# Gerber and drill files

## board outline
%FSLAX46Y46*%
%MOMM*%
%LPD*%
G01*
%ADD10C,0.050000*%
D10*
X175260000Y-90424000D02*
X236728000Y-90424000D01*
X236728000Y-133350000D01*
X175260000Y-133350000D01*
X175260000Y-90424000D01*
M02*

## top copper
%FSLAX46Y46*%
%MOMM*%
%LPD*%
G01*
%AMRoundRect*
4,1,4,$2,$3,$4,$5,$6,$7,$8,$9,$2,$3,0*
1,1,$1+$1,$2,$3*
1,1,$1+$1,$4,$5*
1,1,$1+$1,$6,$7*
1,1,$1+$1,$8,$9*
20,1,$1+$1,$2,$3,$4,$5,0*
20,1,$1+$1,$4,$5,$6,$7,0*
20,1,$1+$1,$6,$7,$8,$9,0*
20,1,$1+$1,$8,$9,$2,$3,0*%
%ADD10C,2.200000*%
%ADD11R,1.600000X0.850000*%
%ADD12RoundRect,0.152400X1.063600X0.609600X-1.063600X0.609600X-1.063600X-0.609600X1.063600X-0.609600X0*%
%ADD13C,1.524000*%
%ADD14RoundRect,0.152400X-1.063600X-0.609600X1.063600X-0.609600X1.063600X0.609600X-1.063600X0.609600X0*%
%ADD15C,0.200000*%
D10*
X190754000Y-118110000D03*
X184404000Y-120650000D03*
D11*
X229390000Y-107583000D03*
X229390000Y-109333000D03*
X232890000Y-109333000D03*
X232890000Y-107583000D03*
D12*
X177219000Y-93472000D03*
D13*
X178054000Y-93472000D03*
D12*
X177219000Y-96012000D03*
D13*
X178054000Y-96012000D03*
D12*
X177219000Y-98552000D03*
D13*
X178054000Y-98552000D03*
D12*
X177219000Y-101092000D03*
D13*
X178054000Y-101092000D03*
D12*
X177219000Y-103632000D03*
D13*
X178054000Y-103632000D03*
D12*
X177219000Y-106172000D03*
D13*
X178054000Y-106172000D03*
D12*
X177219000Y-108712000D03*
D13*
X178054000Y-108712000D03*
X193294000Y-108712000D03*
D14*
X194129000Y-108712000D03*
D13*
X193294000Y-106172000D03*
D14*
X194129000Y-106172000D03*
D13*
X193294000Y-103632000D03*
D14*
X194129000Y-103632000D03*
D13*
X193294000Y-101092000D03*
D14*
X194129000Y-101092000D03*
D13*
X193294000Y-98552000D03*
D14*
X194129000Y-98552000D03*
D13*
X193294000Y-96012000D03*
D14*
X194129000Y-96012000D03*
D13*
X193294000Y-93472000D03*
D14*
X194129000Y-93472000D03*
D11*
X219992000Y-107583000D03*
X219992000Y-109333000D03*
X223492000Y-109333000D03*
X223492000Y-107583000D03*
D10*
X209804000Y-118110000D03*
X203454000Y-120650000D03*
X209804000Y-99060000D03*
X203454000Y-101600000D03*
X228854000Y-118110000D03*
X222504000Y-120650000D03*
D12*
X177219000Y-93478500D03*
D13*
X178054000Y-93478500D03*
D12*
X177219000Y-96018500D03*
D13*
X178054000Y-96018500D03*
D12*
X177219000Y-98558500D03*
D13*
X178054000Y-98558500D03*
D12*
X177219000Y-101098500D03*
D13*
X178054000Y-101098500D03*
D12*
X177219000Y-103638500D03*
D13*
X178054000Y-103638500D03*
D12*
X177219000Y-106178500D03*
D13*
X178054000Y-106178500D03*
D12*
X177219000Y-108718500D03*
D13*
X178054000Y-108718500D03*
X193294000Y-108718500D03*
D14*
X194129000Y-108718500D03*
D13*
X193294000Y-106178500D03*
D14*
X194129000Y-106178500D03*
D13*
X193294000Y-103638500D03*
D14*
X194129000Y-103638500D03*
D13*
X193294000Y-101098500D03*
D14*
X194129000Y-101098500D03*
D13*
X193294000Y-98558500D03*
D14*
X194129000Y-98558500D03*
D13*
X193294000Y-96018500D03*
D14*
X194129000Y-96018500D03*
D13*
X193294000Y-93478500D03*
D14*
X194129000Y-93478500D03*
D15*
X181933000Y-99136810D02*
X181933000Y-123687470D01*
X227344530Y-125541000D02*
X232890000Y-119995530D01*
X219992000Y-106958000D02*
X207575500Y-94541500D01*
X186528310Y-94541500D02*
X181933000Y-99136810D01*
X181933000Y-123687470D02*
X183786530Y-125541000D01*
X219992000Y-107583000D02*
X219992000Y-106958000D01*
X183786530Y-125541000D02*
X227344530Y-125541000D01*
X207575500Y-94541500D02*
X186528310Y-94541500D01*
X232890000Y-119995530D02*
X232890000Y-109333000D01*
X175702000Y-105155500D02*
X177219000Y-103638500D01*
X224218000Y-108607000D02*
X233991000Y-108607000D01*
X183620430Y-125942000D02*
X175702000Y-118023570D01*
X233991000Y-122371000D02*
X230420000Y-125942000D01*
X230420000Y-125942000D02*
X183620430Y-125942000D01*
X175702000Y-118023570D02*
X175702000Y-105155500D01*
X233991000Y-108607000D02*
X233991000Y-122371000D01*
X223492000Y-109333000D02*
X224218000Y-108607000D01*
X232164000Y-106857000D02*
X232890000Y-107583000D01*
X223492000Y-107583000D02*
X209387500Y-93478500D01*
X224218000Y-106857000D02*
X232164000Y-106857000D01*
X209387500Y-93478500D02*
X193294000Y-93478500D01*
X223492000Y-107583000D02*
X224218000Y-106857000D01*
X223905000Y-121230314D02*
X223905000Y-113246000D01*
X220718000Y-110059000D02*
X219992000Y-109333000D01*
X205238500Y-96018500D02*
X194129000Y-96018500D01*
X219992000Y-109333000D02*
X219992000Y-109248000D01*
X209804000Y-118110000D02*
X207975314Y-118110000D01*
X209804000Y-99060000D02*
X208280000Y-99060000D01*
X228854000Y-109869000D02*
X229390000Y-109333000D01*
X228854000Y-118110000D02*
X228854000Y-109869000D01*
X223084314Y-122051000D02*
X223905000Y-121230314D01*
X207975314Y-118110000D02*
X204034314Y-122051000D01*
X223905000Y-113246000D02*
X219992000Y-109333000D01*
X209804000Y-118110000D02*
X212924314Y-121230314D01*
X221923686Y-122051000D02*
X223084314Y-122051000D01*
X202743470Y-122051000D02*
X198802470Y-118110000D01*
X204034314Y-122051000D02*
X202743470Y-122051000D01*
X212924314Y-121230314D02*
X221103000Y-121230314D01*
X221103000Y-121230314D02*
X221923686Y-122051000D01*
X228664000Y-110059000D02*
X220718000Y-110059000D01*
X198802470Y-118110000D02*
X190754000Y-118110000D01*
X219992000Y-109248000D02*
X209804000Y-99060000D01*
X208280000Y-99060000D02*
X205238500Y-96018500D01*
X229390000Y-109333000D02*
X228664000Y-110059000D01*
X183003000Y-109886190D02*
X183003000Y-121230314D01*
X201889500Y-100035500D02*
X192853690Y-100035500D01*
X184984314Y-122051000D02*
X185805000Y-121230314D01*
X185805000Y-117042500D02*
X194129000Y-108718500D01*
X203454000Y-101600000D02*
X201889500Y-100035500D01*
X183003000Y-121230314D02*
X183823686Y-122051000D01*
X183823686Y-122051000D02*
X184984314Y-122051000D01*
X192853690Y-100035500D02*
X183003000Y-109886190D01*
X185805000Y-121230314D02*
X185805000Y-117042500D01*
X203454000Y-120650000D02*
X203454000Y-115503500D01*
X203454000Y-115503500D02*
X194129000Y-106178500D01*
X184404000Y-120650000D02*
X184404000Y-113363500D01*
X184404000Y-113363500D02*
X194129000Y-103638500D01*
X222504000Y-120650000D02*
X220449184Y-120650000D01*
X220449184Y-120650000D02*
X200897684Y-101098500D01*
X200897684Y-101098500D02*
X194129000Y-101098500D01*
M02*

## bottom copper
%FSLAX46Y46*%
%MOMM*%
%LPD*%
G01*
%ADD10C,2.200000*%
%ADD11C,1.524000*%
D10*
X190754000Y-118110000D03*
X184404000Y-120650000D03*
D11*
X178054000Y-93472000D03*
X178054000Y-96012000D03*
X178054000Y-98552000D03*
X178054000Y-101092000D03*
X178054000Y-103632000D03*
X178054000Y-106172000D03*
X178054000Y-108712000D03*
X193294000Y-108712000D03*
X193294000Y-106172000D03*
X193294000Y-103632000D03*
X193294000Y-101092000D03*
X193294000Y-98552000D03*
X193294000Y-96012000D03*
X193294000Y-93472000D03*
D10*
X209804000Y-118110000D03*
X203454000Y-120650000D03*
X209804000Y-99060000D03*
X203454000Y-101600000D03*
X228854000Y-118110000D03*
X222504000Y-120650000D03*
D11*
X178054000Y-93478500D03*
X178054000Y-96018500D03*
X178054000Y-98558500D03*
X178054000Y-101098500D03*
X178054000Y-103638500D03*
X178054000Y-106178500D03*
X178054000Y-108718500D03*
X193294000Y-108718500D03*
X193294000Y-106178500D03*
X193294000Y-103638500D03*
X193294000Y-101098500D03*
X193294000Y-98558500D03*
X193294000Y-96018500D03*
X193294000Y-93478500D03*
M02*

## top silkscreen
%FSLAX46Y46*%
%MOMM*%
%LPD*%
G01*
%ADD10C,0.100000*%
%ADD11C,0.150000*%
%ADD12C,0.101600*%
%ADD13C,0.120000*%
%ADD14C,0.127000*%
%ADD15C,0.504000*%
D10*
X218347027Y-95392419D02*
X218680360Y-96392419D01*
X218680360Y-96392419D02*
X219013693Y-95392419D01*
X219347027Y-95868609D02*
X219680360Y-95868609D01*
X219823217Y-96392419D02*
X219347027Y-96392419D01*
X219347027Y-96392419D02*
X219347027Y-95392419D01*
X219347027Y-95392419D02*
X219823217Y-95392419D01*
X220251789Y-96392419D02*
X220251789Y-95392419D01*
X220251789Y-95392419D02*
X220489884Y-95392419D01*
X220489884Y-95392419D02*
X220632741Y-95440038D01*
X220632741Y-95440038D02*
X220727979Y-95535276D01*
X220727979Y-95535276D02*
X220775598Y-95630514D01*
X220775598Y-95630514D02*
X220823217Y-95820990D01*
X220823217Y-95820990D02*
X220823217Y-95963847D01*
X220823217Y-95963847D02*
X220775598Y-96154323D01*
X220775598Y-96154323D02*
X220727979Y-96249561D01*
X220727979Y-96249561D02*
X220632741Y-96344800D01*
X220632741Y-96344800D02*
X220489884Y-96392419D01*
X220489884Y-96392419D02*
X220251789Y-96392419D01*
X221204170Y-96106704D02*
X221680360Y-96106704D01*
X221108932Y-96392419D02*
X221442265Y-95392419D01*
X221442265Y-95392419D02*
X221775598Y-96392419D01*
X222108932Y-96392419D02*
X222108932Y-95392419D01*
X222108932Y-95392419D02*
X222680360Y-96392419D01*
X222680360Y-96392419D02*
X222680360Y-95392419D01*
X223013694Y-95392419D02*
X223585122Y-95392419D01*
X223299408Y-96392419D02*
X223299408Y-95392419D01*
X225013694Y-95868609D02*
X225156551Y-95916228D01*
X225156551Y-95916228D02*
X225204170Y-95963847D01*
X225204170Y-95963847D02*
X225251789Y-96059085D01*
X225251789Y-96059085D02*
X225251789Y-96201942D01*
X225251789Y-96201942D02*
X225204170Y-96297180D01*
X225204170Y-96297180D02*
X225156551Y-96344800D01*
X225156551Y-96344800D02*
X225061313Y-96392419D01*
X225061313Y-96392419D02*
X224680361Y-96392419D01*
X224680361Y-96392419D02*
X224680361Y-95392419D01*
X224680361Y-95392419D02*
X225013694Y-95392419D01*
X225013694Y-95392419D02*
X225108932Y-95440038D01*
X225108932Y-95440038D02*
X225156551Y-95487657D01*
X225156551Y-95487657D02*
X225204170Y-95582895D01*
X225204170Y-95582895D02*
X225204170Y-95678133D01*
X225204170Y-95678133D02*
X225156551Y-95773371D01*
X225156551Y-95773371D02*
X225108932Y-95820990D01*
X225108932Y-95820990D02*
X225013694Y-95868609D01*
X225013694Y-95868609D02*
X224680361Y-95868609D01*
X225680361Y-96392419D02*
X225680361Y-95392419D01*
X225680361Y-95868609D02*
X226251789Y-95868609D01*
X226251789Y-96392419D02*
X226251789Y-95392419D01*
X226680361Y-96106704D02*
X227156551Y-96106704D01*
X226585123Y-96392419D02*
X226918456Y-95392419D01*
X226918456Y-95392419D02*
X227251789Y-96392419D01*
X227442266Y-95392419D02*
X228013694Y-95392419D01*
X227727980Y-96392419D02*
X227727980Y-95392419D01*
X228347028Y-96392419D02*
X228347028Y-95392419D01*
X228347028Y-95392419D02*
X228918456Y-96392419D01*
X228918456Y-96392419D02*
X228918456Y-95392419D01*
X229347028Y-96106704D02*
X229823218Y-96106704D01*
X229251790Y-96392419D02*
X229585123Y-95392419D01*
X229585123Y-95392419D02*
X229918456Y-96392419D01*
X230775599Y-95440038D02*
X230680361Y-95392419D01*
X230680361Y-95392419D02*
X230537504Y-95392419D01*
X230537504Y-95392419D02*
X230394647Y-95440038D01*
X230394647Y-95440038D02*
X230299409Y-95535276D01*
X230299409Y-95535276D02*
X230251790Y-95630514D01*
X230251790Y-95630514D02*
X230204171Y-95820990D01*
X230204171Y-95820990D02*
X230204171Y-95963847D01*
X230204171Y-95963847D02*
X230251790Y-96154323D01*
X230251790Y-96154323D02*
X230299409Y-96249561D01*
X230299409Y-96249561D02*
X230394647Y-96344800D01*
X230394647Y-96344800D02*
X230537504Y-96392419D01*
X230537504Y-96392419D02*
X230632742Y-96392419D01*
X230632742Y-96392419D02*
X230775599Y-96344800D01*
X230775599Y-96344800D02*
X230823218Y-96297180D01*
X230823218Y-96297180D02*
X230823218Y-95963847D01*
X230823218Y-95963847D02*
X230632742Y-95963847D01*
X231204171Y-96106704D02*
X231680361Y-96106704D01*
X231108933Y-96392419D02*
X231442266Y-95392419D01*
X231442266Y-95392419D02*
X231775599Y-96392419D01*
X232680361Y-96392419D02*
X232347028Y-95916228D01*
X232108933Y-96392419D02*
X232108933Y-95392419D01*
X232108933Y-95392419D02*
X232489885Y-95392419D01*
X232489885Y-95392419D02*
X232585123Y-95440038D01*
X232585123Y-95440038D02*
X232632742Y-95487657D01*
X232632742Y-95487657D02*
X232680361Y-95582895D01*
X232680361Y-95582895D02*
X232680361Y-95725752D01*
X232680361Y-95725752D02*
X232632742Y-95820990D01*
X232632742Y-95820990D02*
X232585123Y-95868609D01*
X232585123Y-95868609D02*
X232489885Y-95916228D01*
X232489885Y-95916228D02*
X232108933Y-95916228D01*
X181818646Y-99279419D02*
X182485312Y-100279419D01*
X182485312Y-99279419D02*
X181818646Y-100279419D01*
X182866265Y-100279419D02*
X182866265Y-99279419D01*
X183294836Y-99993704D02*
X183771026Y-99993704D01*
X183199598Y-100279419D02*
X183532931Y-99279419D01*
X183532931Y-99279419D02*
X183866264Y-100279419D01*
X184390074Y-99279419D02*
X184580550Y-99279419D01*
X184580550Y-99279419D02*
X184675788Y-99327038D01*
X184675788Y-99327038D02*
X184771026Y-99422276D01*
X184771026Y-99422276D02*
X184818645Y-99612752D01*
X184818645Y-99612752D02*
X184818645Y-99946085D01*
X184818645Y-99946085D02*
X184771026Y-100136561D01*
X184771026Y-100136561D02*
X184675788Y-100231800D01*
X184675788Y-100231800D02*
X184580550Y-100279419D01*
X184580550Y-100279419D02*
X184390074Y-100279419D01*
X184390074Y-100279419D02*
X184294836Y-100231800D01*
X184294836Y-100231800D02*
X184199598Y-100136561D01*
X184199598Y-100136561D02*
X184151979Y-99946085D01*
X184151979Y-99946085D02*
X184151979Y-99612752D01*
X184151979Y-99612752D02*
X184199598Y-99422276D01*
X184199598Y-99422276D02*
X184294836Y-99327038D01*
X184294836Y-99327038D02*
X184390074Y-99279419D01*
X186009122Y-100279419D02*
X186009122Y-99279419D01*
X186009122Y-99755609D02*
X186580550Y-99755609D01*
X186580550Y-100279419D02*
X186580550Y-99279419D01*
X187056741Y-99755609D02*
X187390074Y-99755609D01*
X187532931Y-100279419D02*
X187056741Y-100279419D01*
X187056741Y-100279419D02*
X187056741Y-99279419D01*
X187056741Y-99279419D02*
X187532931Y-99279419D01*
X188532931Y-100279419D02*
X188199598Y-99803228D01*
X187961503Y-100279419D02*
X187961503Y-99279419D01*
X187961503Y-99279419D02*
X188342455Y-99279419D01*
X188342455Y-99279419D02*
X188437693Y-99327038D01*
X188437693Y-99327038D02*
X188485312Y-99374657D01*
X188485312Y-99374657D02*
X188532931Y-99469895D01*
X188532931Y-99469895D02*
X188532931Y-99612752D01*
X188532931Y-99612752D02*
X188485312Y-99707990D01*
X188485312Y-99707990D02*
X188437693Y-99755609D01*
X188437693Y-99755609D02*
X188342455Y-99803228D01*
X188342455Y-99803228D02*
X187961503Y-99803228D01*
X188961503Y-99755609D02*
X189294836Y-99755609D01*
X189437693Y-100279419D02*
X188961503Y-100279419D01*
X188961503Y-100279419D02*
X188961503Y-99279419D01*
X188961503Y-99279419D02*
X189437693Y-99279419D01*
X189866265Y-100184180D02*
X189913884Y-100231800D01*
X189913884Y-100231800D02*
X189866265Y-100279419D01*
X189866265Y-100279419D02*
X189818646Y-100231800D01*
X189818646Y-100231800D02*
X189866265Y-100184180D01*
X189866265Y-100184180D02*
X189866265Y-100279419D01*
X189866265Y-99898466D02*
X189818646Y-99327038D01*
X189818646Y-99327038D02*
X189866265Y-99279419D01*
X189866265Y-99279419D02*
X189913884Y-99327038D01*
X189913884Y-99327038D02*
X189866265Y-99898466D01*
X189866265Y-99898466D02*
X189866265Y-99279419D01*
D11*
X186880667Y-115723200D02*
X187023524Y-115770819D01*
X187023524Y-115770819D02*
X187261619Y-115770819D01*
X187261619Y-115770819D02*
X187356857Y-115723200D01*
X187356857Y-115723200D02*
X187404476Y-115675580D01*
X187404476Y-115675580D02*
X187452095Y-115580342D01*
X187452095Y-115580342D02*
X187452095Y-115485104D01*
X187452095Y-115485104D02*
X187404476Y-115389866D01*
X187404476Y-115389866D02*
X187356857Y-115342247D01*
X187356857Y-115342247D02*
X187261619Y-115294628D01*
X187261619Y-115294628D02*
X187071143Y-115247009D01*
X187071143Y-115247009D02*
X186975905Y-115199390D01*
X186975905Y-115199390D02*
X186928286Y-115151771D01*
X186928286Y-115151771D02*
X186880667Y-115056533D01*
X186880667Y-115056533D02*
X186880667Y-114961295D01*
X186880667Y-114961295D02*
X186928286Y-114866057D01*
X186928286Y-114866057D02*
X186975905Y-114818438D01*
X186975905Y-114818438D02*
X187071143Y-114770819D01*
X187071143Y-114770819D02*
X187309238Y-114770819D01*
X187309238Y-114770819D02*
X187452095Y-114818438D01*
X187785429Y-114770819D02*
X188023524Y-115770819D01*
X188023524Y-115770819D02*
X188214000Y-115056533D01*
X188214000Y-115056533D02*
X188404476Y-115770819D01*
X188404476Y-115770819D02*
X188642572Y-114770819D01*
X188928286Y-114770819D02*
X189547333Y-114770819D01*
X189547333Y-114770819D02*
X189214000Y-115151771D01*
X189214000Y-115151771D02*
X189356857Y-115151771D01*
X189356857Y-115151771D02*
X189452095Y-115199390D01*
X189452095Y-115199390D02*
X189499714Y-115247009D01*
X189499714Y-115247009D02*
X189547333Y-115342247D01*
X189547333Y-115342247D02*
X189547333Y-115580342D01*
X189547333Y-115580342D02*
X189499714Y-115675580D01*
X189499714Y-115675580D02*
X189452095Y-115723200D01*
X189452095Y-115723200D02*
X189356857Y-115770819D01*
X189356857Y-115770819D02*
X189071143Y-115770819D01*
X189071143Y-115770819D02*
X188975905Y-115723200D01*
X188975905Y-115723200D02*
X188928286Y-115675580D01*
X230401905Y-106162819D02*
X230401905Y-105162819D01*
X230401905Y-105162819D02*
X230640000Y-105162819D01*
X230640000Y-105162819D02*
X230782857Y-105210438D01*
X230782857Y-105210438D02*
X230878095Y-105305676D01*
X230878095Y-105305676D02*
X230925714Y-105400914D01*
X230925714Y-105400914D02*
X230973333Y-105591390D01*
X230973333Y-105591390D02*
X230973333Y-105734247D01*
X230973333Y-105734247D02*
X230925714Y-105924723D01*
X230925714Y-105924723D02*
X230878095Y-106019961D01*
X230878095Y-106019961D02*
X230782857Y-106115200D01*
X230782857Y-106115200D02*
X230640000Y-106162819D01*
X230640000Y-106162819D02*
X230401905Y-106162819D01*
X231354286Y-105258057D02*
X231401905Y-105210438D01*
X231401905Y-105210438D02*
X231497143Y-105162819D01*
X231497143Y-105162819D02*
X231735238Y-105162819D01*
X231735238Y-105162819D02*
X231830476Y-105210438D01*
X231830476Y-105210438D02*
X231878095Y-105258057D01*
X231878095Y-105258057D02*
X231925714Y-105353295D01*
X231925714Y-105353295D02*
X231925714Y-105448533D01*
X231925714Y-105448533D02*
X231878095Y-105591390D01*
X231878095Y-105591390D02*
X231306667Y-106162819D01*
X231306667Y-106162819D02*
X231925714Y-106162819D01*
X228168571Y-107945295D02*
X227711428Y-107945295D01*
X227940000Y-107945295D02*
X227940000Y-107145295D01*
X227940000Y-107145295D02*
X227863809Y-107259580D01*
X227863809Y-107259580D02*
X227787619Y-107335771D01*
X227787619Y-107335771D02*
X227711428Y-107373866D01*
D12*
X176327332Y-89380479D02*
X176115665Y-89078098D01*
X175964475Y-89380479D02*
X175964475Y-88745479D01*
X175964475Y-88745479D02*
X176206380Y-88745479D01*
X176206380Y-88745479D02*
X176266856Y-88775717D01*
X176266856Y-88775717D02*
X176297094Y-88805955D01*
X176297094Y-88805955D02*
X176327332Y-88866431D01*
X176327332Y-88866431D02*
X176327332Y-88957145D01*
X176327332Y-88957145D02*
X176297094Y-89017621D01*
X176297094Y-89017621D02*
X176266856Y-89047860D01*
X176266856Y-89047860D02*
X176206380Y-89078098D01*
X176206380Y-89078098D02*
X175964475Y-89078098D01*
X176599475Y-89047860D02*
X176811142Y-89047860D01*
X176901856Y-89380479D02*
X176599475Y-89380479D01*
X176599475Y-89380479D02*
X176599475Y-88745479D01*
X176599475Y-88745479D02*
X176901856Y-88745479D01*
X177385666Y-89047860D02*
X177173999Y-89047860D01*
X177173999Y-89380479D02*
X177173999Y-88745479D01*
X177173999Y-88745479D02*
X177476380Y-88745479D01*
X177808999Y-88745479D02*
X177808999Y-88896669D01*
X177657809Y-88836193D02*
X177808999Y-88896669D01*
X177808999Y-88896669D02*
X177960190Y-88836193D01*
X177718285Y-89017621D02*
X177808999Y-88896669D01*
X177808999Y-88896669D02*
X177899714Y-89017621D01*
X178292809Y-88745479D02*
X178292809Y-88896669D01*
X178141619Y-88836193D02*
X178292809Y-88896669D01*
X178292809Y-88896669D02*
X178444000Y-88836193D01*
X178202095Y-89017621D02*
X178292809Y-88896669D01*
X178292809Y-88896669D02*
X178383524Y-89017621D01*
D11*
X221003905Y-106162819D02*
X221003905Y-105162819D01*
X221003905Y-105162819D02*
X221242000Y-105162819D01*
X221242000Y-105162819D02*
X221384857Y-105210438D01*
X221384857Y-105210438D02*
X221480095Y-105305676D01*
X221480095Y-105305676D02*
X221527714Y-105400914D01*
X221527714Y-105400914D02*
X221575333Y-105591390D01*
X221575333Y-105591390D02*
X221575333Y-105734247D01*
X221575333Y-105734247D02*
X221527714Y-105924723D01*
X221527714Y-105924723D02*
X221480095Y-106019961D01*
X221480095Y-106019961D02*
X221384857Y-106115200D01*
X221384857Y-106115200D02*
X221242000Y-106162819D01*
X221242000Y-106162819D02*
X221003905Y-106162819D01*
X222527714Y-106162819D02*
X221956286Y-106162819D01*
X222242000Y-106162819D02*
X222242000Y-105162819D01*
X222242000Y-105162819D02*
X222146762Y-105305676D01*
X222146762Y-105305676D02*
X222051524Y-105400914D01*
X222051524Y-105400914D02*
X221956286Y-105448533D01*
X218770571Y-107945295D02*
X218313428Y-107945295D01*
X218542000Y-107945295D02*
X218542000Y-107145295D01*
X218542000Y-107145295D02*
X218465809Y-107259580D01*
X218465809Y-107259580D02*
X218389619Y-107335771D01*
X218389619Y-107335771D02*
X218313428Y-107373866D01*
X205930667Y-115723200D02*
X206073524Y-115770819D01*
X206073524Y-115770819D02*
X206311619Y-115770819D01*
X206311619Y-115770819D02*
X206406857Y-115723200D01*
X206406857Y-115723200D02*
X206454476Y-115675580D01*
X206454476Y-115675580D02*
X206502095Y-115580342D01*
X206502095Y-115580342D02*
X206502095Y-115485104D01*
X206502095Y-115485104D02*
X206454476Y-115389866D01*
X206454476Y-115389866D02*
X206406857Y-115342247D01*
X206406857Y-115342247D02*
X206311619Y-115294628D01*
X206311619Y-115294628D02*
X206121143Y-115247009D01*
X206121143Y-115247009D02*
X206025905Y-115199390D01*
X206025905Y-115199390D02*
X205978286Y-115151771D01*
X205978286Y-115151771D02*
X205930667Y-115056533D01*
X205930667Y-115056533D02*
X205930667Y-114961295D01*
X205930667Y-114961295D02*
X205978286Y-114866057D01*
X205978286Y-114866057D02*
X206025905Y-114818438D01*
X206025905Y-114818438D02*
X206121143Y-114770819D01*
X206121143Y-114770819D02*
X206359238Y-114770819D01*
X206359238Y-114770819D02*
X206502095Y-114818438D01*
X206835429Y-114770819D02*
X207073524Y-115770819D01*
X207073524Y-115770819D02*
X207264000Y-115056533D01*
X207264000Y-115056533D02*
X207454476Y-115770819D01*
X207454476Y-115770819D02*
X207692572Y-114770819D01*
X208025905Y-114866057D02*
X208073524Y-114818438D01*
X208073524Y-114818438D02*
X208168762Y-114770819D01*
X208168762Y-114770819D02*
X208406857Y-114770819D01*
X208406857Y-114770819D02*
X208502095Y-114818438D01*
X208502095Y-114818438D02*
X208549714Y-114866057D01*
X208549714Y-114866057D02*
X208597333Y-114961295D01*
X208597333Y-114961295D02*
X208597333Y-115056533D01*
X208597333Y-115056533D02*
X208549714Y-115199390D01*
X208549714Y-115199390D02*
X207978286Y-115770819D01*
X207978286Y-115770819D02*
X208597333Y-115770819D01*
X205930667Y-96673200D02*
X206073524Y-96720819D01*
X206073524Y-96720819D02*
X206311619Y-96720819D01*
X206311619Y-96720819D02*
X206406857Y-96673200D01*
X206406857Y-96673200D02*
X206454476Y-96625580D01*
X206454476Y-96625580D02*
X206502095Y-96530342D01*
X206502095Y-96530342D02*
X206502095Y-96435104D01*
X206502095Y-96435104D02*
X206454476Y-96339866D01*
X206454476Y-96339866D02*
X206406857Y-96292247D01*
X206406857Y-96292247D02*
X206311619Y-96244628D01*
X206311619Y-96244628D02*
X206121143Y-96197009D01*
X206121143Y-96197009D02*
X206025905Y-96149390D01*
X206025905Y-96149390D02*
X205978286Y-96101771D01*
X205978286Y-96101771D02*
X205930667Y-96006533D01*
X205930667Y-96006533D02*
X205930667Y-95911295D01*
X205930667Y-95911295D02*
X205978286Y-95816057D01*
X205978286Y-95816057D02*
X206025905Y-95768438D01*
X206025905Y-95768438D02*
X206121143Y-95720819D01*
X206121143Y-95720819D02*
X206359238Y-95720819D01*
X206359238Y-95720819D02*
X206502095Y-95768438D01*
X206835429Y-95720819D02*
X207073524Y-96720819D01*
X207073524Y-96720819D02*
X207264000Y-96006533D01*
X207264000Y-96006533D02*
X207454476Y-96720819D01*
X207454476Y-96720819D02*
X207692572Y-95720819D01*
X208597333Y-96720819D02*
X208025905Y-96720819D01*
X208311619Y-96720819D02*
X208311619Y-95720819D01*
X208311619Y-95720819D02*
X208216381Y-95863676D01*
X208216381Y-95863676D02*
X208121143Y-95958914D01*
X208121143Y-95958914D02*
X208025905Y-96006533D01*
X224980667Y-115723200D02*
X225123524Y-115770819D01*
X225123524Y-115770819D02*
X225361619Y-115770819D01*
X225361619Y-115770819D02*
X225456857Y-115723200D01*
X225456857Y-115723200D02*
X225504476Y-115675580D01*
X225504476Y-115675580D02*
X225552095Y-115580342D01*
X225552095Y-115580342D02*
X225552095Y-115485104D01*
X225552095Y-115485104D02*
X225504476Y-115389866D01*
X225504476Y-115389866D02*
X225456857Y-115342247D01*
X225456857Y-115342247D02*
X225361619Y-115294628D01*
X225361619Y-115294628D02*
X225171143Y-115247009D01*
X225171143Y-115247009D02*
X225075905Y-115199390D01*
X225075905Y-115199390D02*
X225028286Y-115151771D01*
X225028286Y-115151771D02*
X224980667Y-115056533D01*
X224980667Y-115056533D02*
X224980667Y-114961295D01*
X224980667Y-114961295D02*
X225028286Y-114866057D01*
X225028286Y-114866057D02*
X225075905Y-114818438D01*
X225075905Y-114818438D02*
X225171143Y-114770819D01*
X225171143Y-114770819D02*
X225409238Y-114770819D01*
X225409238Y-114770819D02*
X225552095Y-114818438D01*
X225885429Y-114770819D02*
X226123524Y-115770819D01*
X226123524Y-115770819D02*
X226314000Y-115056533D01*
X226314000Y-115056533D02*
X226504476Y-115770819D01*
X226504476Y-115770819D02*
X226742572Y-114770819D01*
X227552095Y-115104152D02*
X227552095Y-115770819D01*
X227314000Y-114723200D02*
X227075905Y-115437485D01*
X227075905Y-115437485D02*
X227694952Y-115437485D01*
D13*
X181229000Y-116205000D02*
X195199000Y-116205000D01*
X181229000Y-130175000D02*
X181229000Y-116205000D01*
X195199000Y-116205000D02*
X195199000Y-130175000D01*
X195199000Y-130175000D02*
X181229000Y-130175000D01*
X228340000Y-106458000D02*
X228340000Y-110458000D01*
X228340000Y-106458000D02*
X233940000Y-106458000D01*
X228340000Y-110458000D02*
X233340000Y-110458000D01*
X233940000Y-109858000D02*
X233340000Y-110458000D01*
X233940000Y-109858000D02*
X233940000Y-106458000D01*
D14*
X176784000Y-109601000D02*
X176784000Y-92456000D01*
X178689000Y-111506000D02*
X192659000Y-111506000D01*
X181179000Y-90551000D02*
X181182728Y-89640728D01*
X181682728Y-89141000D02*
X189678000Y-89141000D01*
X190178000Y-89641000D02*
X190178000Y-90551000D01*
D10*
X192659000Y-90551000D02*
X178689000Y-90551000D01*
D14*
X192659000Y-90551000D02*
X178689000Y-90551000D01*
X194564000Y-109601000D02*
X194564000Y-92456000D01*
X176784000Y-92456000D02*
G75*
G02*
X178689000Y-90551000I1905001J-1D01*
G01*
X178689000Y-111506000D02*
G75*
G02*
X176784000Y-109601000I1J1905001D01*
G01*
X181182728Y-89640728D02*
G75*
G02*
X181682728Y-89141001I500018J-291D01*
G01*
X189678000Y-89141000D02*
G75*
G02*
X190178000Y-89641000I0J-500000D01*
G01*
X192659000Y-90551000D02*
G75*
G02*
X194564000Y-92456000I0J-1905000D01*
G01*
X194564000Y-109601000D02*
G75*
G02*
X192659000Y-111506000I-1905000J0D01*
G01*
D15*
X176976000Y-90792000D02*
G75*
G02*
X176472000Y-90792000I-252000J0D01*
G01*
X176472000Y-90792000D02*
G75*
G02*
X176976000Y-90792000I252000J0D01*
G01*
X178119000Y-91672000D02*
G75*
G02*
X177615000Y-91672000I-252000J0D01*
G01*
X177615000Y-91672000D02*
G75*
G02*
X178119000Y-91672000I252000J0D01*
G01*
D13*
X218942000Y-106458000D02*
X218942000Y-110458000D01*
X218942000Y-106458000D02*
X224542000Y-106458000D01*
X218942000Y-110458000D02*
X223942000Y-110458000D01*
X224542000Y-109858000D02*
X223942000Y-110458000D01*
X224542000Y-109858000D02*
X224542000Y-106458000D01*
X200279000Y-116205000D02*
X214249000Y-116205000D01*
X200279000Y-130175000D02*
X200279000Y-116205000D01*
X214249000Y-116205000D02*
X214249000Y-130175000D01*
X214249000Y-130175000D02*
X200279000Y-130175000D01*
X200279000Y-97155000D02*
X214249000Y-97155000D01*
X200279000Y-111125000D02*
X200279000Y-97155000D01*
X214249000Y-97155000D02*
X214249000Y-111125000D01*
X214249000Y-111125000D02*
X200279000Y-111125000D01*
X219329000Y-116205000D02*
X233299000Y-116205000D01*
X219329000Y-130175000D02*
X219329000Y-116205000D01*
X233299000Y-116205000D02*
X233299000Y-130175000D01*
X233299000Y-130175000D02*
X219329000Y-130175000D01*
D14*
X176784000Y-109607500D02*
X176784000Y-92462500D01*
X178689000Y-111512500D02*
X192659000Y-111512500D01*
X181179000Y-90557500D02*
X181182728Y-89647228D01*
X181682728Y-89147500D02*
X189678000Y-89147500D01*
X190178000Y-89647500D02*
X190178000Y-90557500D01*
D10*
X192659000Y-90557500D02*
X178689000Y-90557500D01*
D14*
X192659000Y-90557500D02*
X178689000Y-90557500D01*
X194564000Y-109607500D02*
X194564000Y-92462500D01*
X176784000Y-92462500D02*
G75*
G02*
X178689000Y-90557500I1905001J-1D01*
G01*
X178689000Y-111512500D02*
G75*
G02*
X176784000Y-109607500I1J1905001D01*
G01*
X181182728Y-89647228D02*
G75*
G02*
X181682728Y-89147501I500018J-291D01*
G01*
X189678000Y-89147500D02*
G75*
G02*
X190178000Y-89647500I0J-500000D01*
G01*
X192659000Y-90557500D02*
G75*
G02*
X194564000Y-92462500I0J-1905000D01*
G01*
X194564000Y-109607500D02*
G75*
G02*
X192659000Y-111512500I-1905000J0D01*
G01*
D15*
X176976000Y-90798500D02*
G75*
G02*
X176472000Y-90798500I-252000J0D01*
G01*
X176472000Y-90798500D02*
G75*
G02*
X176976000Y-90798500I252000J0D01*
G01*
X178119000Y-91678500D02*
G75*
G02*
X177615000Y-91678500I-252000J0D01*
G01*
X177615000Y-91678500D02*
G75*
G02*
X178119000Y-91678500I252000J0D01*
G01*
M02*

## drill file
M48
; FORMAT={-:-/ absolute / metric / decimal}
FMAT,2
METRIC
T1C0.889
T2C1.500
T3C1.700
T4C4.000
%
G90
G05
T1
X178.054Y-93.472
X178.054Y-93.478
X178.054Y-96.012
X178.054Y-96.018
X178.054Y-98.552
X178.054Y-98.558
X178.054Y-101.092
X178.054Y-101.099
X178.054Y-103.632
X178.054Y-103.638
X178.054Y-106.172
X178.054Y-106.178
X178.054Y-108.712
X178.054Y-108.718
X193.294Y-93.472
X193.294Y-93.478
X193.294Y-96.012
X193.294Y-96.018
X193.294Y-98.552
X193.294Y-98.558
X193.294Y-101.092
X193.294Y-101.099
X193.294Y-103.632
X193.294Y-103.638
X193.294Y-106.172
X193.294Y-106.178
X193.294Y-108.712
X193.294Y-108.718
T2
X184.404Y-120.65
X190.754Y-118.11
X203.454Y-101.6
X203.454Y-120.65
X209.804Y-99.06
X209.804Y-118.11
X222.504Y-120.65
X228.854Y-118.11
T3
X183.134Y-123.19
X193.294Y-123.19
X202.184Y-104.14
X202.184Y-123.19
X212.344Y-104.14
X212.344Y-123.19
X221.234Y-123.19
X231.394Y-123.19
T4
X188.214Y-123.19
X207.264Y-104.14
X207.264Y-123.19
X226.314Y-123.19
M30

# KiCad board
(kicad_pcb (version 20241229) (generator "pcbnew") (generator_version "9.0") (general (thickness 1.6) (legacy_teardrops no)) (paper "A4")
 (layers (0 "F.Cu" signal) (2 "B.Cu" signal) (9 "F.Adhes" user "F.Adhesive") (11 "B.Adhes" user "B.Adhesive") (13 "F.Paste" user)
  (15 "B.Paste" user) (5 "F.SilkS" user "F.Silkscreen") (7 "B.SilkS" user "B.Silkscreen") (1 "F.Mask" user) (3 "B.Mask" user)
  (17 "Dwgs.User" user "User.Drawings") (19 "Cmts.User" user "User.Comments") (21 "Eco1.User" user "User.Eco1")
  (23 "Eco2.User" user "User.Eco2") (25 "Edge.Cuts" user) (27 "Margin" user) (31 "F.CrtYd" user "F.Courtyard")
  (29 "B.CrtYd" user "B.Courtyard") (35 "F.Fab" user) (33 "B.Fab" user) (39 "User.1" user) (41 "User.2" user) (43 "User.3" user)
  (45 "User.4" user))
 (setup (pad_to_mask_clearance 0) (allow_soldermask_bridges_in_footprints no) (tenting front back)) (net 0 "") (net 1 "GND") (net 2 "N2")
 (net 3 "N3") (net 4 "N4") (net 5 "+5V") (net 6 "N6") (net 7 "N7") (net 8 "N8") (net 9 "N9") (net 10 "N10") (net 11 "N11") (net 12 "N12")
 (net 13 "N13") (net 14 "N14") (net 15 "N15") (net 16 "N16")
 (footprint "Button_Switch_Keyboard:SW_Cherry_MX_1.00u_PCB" (layer "F.Cu") (at 190.754 118.11)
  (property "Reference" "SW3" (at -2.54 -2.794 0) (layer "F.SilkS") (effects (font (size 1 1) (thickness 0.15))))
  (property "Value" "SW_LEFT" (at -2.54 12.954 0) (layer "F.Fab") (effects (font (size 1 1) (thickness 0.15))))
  (fp_line (start -9.525 -1.905) (end 4.445 -1.905) (stroke (width 0.12) (type solid)) (layer "F.SilkS"))
  (fp_line (start -9.525 12.065) (end -9.525 -1.905) (stroke (width 0.12) (type solid)) (layer "F.SilkS"))
  (fp_line (start 4.445 -1.905) (end 4.445 12.065) (stroke (width 0.12) (type solid)) (layer "F.SilkS"))
  (fp_line (start 4.445 12.065) (end -9.525 12.065) (stroke (width 0.12) (type solid)) (layer "F.SilkS"))
  (pad "" np_thru_hole circle (at -7.62 5.08) (size 1.7 1.7) (drill 1.7) (layers "*.Cu" "*.Mask"))
  (pad "" np_thru_hole circle (at -2.54 5.08) (size 4 4) (drill 4) (layers "*.Cu" "*.Mask"))
  (pad "" np_thru_hole circle (at 2.54 5.08) (size 1.7 1.7) (drill 1.7) (layers "*.Cu" "*.Mask"))
  (pad "1" thru_hole circle (at 0 0) (size 2.2 2.2) (drill 1.5) (layers "*.Cu" "*.Mask") (remove_unused_layers no) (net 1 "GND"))
  (pad "2" thru_hole circle (at -6.35 2.54) (size 2.2 2.2) (drill 1.5) (layers "*.Cu" "*.Mask") (remove_unused_layers no) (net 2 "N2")))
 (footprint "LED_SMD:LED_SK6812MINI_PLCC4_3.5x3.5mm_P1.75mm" (layer "F.Cu") (at 231.14 108.458)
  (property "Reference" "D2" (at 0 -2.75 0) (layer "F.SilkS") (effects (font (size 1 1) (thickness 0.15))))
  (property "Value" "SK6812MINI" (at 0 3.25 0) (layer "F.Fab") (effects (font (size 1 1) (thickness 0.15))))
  (fp_line (start -2.8 -2) (end -2.8 2) (stroke (width 0.12) (type default)) (layer "F.SilkS"))
  (fp_line (start -2.8 -2) (end 2.8 -2) (stroke (width 0.12) (type solid)) (layer "F.SilkS"))
  (fp_line (start -2.8 2) (end 2.2 2) (stroke (width 0.12) (type solid)) (layer "F.SilkS"))
  (fp_line (start 2.8 1.4) (end 2.2 2) (stroke (width 0.12) (type default)) (layer "F.SilkS"))
  (fp_line (start 2.8 1.4) (end 2.8 -2) (stroke (width 0.12) (type solid)) (layer "F.SilkS"))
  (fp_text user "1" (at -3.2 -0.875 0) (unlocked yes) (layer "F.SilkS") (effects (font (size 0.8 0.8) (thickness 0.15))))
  (pad "1" smd rect (at -1.75 -0.875) (size 1.6 0.85) (layers "F.Cu" "F.Mask" "F.Paste") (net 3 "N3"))
  (pad "2" smd rect (at -1.75 0.875) (size 1.6 0.85) (layers "F.Cu" "F.Mask" "F.Paste") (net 1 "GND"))
  (pad "3" smd rect (at 1.75 0.875) (size 1.6 0.85) (layers "F.Cu" "F.Mask" "F.Paste") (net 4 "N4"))
  (pad "4" smd rect (at 1.75 -0.875) (size 1.6 0.85) (layers "F.Cu" "F.Mask" "F.Paste") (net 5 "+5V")))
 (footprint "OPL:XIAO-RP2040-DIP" (layer "F.Cu") (at 185.674 101.092)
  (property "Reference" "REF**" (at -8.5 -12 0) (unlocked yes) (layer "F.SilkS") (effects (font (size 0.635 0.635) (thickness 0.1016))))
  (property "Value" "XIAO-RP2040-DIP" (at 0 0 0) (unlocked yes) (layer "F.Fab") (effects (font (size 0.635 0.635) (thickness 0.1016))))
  (fp_line (start -8.89 8.509) (end -8.89 -8.636) (stroke (width 0.127) (type solid)) (layer "F.SilkS"))
  (fp_line (start -6.985 10.414) (end 6.985 10.414) (stroke (width 0.127) (type solid)) (layer "F.SilkS"))
  (fp_line (start -4.495 -10.541) (end -4.491272 -11.451272) (stroke (width 0.127) (type solid)) (layer "F.SilkS"))
  (fp_line (start -3.991272 -11.951) (end 4.004 -11.951) (stroke (width 0.127) (type solid)) (layer "F.SilkS"))
  (fp_line (start 4.504 -11.451) (end 4.504 -10.541) (stroke (width 0.127) (type solid)) (layer "F.SilkS"))
  (fp_line (start 6.985 -10.541) (end -6.985 -10.541) (stroke (width 0.1) (type solid)) (layer "F.SilkS"))
  (fp_line (start 6.985 -10.541) (end -6.985 -10.541) (stroke (width 0.127) (type solid)) (layer "F.SilkS"))
  (fp_line (start 8.89 8.509) (end 8.89 -8.636) (stroke (width 0.127) (type solid)) (layer "F.SilkS"))
  (fp_arc (start -8.89 -8.636) (mid -8.332038 -9.983038) (end -6.985 -10.541) (stroke (width 0.127) (type solid)) (layer "F.SilkS"))
  (fp_arc (start -6.985 10.414) (mid -8.332038 9.856038) (end -8.89 8.509) (stroke (width 0.127) (type solid)) (layer "F.SilkS"))
  (fp_arc (start -4.491272 -11.451272) (mid -4.344728 -11.80464) (end -3.991272 -11.951) (stroke (width 0.127) (type default))
   (layer "F.SilkS"))
  (fp_arc (start 4.004 -11.951) (mid 4.357553 -11.804553) (end 4.504 -11.451) (stroke (width 0.127) (type default)) (layer "F.SilkS"))
  (fp_arc (start 6.985 -10.541) (mid 8.332038 -9.983038) (end 8.89 -8.636) (stroke (width 0.127) (type solid)) (layer "F.SilkS"))
  (fp_arc (start 8.89 8.509) (mid 8.332038 9.856038) (end 6.985 10.414) (stroke (width 0.127) (type solid)) (layer "F.SilkS"))
  (fp_circle (center -8.95 -10.3) (end -8.95 -10.554) (stroke (width 0.5) (type solid)) (fill yes) (layer "F.SilkS"))
  (fp_circle (center -7.807 -9.42) (end -7.807 -9.674) (stroke (width 0.5) (type solid)) (fill yes) (layer "F.SilkS"))
  (pad "1" smd roundrect (at -8.455 -7.62 180) (size 2.432 1.524) (layers "F.Cu" "F.Mask") (roundrect_rratio 0.1) (thermal_bridge_angle 45))
  (pad "1" thru_hole circle (at -7.62 -7.62 180) (size 1.524 1.524) (drill 0.889) (layers "*.Cu" "*.Mask") (remove_unused_layers no))
  (pad "2" smd roundrect (at -8.455 -5.08 180) (size 2.432 1.524) (layers "F.Cu" "F.Mask") (roundrect_rratio 0.1) (thermal_bridge_angle 45))
  (pad "2" thru_hole circle (at -7.62 -5.08 180) (size 1.524 1.524) (drill 0.889) (layers "*.Cu" "*.Mask") (remove_unused_layers no))
  (pad "3" smd roundrect (at -8.455 -2.54 180) (size 2.432 1.524) (layers "F.Cu" "F.Mask") (roundrect_rratio 0.1) (thermal_bridge_angle 45))
  (pad "3" thru_hole circle (at -7.62 -2.54 180) (size 1.524 1.524) (drill 0.889) (layers "*.Cu" "*.Mask") (remove_unused_layers no))
  (pad "4" smd roundrect (at -8.455 0 180) (size 2.432 1.524) (layers "F.Cu" "F.Mask") (roundrect_rratio 0.1) (thermal_bridge_angle 45))
  (pad "4" thru_hole circle (at -7.62 0 180) (size 1.524 1.524) (drill 0.889) (layers "*.Cu" "*.Mask") (remove_unused_layers no))
  (pad "5" smd roundrect (at -8.455 2.54 180) (size 2.432 1.524) (layers "F.Cu" "F.Mask") (roundrect_rratio 0.1) (thermal_bridge_angle 45))
  (pad "5" thru_hole circle (at -7.62 2.54 180) (size 1.524 1.524) (drill 0.889) (layers "*.Cu" "*.Mask") (remove_unused_layers no))
  (pad "6" smd roundrect (at -8.455 5.08 180) (size 2.432 1.524) (layers "F.Cu" "F.Mask") (roundrect_rratio 0.1) (thermal_bridge_angle 45))
  (pad "6" thru_hole circle (at -7.62 5.08 180) (size 1.524 1.524) (drill 0.889) (layers "*.Cu" "*.Mask") (remove_unused_layers no))
  (pad "7" smd roundrect (at -8.455 7.62 180) (size 2.432 1.524) (layers "F.Cu" "F.Mask") (roundrect_rratio 0.1) (thermal_bridge_angle 45))
  (pad "7" thru_hole circle (at -7.62 7.62 180) (size 1.524 1.524) (drill 0.889) (layers "*.Cu" "*.Mask") (remove_unused_layers no))
  (pad "8" thru_hole circle (at 7.62 7.62) (size 1.524 1.524) (drill 0.889) (layers "*.Cu" "*.Mask") (remove_unused_layers no))
  (pad "8" smd roundrect (at 8.455 7.62) (size 2.432 1.524) (layers "F.Cu" "F.Mask") (roundrect_rratio 0.1) (thermal_bridge_angle 45))
  (pad "9" thru_hole circle (at 7.62 5.08) (size 1.524 1.524) (drill 0.889) (layers "*.Cu" "*.Mask") (remove_unused_layers no))
  (pad "9" smd roundrect (at 8.455 5.08) (size 2.432 1.524) (layers "F.Cu" "F.Mask") (roundrect_rratio 0.1) (thermal_bridge_angle 45))
  (pad "10" thru_hole circle (at 7.62 2.54) (size 1.524 1.524) (drill 0.889) (layers "*.Cu" "*.Mask") (remove_unused_layers no))
  (pad "10" smd roundrect (at 8.455 2.54) (size 2.432 1.524) (layers "F.Cu" "F.Mask") (roundrect_rratio 0.1) (thermal_bridge_angle 45))
  (pad "11" thru_hole circle (at 7.62 0) (size 1.524 1.524) (drill 0.889) (layers "*.Cu" "*.Mask") (remove_unused_layers no))
  (pad "11" smd roundrect (at 8.455 0) (size 2.432 1.524) (layers "F.Cu" "F.Mask") (roundrect_rratio 0.1) (thermal_bridge_angle 45))
  (pad "12" thru_hole circle (at 7.62 -2.54) (size 1.524 1.524) (drill 0.889) (layers "*.Cu" "*.Mask") (remove_unused_layers no))
  (pad "12" smd roundrect (at 8.455 -2.54) (size 2.432 1.524) (layers "F.Cu" "F.Mask") (roundrect_rratio 0.1) (thermal_bridge_angle 45))
  (pad "13" thru_hole circle (at 7.62 -5.08) (size 1.524 1.524) (drill 0.889) (layers "*.Cu" "*.Mask") (remove_unused_layers no))
  (pad "13" smd roundrect (at 8.455 -5.08) (size 2.432 1.524) (layers "F.Cu" "F.Mask") (roundrect_rratio 0.1) (thermal_bridge_angle 45))
  (pad "14" thru_hole circle (at 7.62 -7.62) (size 1.524 1.524) (drill 0.889) (layers "*.Cu" "*.Mask") (remove_unused_layers no))
  (pad "14" smd roundrect (at 8.455 -7.62) (size 2.432 1.524) (layers "F.Cu" "F.Mask") (roundrect_rratio 0.1) (thermal_bridge_angle 45)))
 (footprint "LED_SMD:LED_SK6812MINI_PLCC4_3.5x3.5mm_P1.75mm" (layer "F.Cu") (at 221.742 108.458)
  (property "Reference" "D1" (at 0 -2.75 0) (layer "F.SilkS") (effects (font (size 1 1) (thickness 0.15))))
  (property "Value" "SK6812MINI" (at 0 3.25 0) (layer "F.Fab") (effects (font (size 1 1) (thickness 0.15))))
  (fp_line (start -2.8 -2) (end -2.8 2) (stroke (width 0.12) (type default)) (layer "F.SilkS"))
  (fp_line (start -2.8 -2) (end 2.8 -2) (stroke (width 0.12) (type solid)) (layer "F.SilkS"))
  (fp_line (start -2.8 2) (end 2.2 2) (stroke (width 0.12) (type solid)) (layer "F.SilkS"))
  (fp_line (start 2.8 1.4) (end 2.2 2) (stroke (width 0.12) (type default)) (layer "F.SilkS"))
  (fp_line (start 2.8 1.4) (end 2.8 -2) (stroke (width 0.12) (type solid)) (layer "F.SilkS"))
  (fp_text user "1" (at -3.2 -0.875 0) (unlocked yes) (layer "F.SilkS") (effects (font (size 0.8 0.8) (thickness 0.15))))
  (pad "1" smd rect (at -1.75 -0.875) (size 1.6 0.85) (layers "F.Cu" "F.Mask" "F.Paste") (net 4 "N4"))
  (pad "2" smd rect (at -1.75 0.875) (size 1.6 0.85) (layers "F.Cu" "F.Mask" "F.Paste") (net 1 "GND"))
  (pad "3" smd rect (at 1.75 0.875) (size 1.6 0.85) (layers "F.Cu" "F.Mask" "F.Paste") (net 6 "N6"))
  (pad "4" smd rect (at 1.75 -0.875) (size 1.6 0.85) (layers "F.Cu" "F.Mask" "F.Paste") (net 5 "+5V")))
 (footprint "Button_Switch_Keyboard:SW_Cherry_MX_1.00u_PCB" (layer "F.Cu") (at 209.804 118.11)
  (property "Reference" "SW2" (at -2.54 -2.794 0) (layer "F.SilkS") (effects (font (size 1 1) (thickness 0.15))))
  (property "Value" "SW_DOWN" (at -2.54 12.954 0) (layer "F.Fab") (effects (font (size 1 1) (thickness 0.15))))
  (fp_line (start -9.525 -1.905) (end 4.445 -1.905) (stroke (width 0.12) (type solid)) (layer "F.SilkS"))
  (fp_line (start -9.525 12.065) (end -9.525 -1.905) (stroke (width 0.12) (type solid)) (layer "F.SilkS"))
  (fp_line (start 4.445 -1.905) (end 4.445 12.065) (stroke (width 0.12) (type solid)) (layer "F.SilkS"))
  (fp_line (start 4.445 12.065) (end -9.525 12.065) (stroke (width 0.12) (type solid)) (layer "F.SilkS"))
  (pad "" np_thru_hole circle (at -7.62 5.08) (size 1.7 1.7) (drill 1.7) (layers "*.Cu" "*.Mask"))
  (pad "" np_thru_hole circle (at -2.54 5.08) (size 4 4) (drill 4) (layers "*.Cu" "*.Mask"))
  (pad "" np_thru_hole circle (at 2.54 5.08) (size 1.7 1.7) (drill 1.7) (layers "*.Cu" "*.Mask"))
  (pad "1" thru_hole circle (at 0 0) (size 2.2 2.2) (drill 1.5) (layers "*.Cu" "*.Mask") (remove_unused_layers no) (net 1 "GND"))
  (pad "2" thru_hole circle (at -6.35 2.54) (size 2.2 2.2) (drill 1.5) (layers "*.Cu" "*.Mask") (remove_unused_layers no) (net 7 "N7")))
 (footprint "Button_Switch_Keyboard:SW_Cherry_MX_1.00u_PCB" (layer "F.Cu") (at 209.804 99.06)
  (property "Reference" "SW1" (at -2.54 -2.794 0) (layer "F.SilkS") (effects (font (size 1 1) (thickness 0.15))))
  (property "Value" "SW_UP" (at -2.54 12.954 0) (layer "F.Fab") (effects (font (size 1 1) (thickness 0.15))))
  (fp_line (start -9.525 -1.905) (end 4.445 -1.905) (stroke (width 0.12) (type solid)) (layer "F.SilkS"))
  (fp_line (start -9.525 12.065) (end -9.525 -1.905) (stroke (width 0.12) (type solid)) (layer "F.SilkS"))
  (fp_line (start 4.445 -1.905) (end 4.445 12.065) (stroke (width 0.12) (type solid)) (layer "F.SilkS"))
  (fp_line (start 4.445 12.065) (end -9.525 12.065) (stroke (width 0.12) (type solid)) (layer "F.SilkS"))
  (pad "" np_thru_hole circle (at -7.62 5.08) (size 1.7 1.7) (drill 1.7) (layers "*.Cu" "*.Mask"))
  (pad "" np_thru_hole circle (at -2.54 5.08) (size 4 4) (drill 4) (layers "*.Cu" "*.Mask"))
  (pad "" np_thru_hole circle (at 2.54 5.08) (size 1.7 1.7) (drill 1.7) (layers "*.Cu" "*.Mask"))
  (pad "1" thru_hole circle (at 0 0) (size 2.2 2.2) (drill 1.5) (layers "*.Cu" "*.Mask") (remove_unused_layers no) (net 1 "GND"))
  (pad "2" thru_hole circle (at -6.35 2.54) (size 2.2 2.2) (drill 1.5) (layers "*.Cu" "*.Mask") (remove_unused_layers no) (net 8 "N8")))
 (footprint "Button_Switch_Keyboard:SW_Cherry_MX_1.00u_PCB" (layer "F.Cu") (at 228.854 118.11)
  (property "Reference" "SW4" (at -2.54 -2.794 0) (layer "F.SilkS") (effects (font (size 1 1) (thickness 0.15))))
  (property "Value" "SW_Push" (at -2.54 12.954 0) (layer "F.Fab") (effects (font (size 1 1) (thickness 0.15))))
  (fp_line (start -9.525 -1.905) (end 4.445 -1.905) (stroke (width 0.12) (type solid)) (layer "F.SilkS"))
  (fp_line (start -9.525 12.065) (end -9.525 -1.905) (stroke (width 0.12) (type solid)) (layer "F.SilkS"))
  (fp_line (start 4.445 -1.905) (end 4.445 12.065) (stroke (width 0.12) (type solid)) (layer "F.SilkS"))
  (fp_line (start 4.445 12.065) (end -9.525 12.065) (stroke (width 0.12) (type solid)) (layer "F.SilkS"))
  (pad "" np_thru_hole circle (at -7.62 5.08) (size 1.7 1.7) (drill 1.7) (layers "*.Cu" "*.Mask"))
  (pad "" np_thru_hole circle (at -2.54 5.08) (size 4 4) (drill 4) (layers "*.Cu" "*.Mask"))
  (pad "" np_thru_hole circle (at 2.54 5.08) (size 1.7 1.7) (drill 1.7) (layers "*.Cu" "*.Mask"))
  (pad "1" thru_hole circle (at 0 0) (size 2.2 2.2) (drill 1.5) (layers "*.Cu" "*.Mask") (remove_unused_layers no) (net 1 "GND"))
  (pad "2" thru_hole circle (at -6.35 2.54) (size 2.2 2.2) (drill 1.5) (layers "*.Cu" "*.Mask") (remove_unused_layers no) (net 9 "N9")))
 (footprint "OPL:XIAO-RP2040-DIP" (layer "F.Cu") (at 185.674 101.0985)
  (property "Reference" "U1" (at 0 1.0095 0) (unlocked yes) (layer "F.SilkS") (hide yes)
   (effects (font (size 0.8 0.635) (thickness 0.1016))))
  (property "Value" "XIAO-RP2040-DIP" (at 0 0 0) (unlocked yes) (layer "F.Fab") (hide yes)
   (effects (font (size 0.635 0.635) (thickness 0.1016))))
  (fp_line (start -8.89 8.509) (end -8.89 -8.636) (stroke (width 0.127) (type solid)) (layer "F.SilkS"))
  (fp_line (start -6.985 10.414) (end 6.985 10.414) (stroke (width 0.127) (type solid)) (layer "F.SilkS"))
  (fp_line (start -4.495 -10.541) (end -4.491272 -11.451272) (stroke (width 0.127) (type solid)) (layer "F.SilkS"))
  (fp_line (start -3.991272 -11.951) (end 4.004 -11.951) (stroke (width 0.127) (type solid)) (layer "F.SilkS"))
  (fp_line (start 4.504 -11.451) (end 4.504 -10.541) (stroke (width 0.127) (type solid)) (layer "F.SilkS"))
  (fp_line (start 6.985 -10.541) (end -6.985 -10.541) (stroke (width 0.1) (type solid)) (layer "F.SilkS"))
  (fp_line (start 6.985 -10.541) (end -6.985 -10.541) (stroke (width 0.127) (type solid)) (layer "F.SilkS"))
  (fp_line (start 8.89 8.509) (end 8.89 -8.636) (stroke (width 0.127) (type solid)) (layer "F.SilkS"))
  (fp_arc (start -8.89 -8.636) (mid -8.332038 -9.983038) (end -6.985 -10.541) (stroke (width 0.127) (type solid)) (layer "F.SilkS"))
  (fp_arc (start -6.985 10.414) (mid -8.332038 9.856038) (end -8.89 8.509) (stroke (width 0.127) (type solid)) (layer "F.SilkS"))
  (fp_arc (start -4.491272 -11.451272) (mid -4.344728 -11.80464) (end -3.991272 -11.951) (stroke (width 0.127) (type default))
   (layer "F.SilkS"))
  (fp_arc (start 4.004 -11.951) (mid 4.357553 -11.804553) (end 4.504 -11.451) (stroke (width 0.127) (type default)) (layer "F.SilkS"))
  (fp_arc (start 6.985 -10.541) (mid 8.332038 -9.983038) (end 8.89 -8.636) (stroke (width 0.127) (type solid)) (layer "F.SilkS"))
  (fp_arc (start 8.89 8.509) (mid 8.332038 9.856038) (end 6.985 10.414) (stroke (width 0.127) (type solid)) (layer "F.SilkS"))
  (fp_circle (center -8.95 -10.3) (end -8.95 -10.554) (stroke (width 0.5) (type solid)) (fill yes) (layer "F.SilkS"))
  (fp_circle (center -7.807 -9.42) (end -7.807 -9.674) (stroke (width 0.5) (type solid)) (fill yes) (layer "F.SilkS"))
  (pad "1" smd roundrect (at -8.455 -7.62 180) (size 2.432 1.524) (layers "F.Cu" "F.Mask") (roundrect_rratio 0.1) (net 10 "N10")
   (thermal_bridge_angle 45))
  (pad "1" thru_hole circle (at -7.62 -7.62 180) (size 1.524 1.524) (drill 0.889) (layers "*.Cu" "*.Mask") (remove_unused_layers no)
   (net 10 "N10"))
  (pad "2" smd roundrect (at -8.455 -5.08 180) (size 2.432 1.524) (layers "F.Cu" "F.Mask") (roundrect_rratio 0.1) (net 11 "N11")
   (thermal_bridge_angle 45))
  (pad "2" thru_hole circle (at -7.62 -5.08 180) (size 1.524 1.524) (drill 0.889) (layers "*.Cu" "*.Mask") (remove_unused_layers no)
   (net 11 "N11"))
  (pad "3" smd roundrect (at -8.455 -2.54 180) (size 2.432 1.524) (layers "F.Cu" "F.Mask") (roundrect_rratio 0.1) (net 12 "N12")
   (thermal_bridge_angle 45))
  (pad "3" thru_hole circle (at -7.62 -2.54 180) (size 1.524 1.524) (drill 0.889) (layers "*.Cu" "*.Mask") (remove_unused_layers no)
   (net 12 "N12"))
  (pad "4" smd roundrect (at -8.455 0 180) (size 2.432 1.524) (layers "F.Cu" "F.Mask") (roundrect_rratio 0.1) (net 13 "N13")
   (thermal_bridge_angle 45))
  (pad "4" thru_hole circle (at -7.62 0 180) (size 1.524 1.524) (drill 0.889) (layers "*.Cu" "*.Mask") (remove_unused_layers no)
   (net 13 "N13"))
  (pad "5" smd roundrect (at -8.455 2.54 180) (size 2.432 1.524) (layers "F.Cu" "F.Mask") (roundrect_rratio 0.1) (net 6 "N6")
   (thermal_bridge_angle 45))
  (pad "5" thru_hole circle (at -7.62 2.54 180) (size 1.524 1.524) (drill 0.889) (layers "*.Cu" "*.Mask") (remove_unused_layers no)
   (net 6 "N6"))
  (pad "6" smd roundrect (at -8.455 5.08 180) (size 2.432 1.524) (layers "F.Cu" "F.Mask") (roundrect_rratio 0.1) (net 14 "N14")
   (thermal_bridge_angle 45))
  (pad "6" thru_hole circle (at -7.62 5.08 180) (size 1.524 1.524) (drill 0.889) (layers "*.Cu" "*.Mask") (remove_unused_layers no)
   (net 14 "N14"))
  (pad "7" smd roundrect (at -8.455 7.62 180) (size 2.432 1.524) (layers "F.Cu" "F.Mask") (roundrect_rratio 0.1) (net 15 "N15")
   (thermal_bridge_angle 45))
  (pad "7" thru_hole circle (at -7.62 7.62 180) (size 1.524 1.524) (drill 0.889) (layers "*.Cu" "*.Mask") (remove_unused_layers no)
   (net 15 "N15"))
  (pad "8" thru_hole circle (at 7.62 7.62) (size 1.524 1.524) (drill 0.889) (layers "*.Cu" "*.Mask") (remove_unused_layers no) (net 8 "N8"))
  (pad "8" smd roundrect (at 8.455 7.62) (size 2.432 1.524) (layers "F.Cu" "F.Mask") (roundrect_rratio 0.1) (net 8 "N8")
   (thermal_bridge_angle 45))
  (pad "9" thru_hole circle (at 7.62 5.08) (size 1.524 1.524) (drill 0.889) (layers "*.Cu" "*.Mask") (remove_unused_layers no) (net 7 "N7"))
  (pad "9" smd roundrect (at 8.455 5.08) (size 2.432 1.524) (layers "F.Cu" "F.Mask") (roundrect_rratio 0.1) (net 7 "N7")
   (thermal_bridge_angle 45))
  (pad "10" thru_hole circle (at 7.62 2.54) (size 1.524 1.524) (drill 0.889) (layers "*.Cu" "*.Mask") (remove_unused_layers no) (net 2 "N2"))
  (pad "10" smd roundrect (at 8.455 2.54) (size 2.432 1.524) (layers "F.Cu" "F.Mask") (roundrect_rratio 0.1) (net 2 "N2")
   (thermal_bridge_angle 45))
  (pad "11" thru_hole circle (at 7.62 0) (size 1.524 1.524) (drill 0.889) (layers "*.Cu" "*.Mask") (remove_unused_layers no) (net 9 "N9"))
  (pad "11" smd roundrect (at 8.455 0) (size 2.432 1.524) (layers "F.Cu" "F.Mask") (roundrect_rratio 0.1) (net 9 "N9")
   (thermal_bridge_angle 45))
  (pad "12" thru_hole circle (at 7.62 -2.54) (size 1.524 1.524) (drill 0.889) (layers "*.Cu" "*.Mask") (remove_unused_layers no)
   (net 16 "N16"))
  (pad "12" smd roundrect (at 8.455 -2.54) (size 2.432 1.524) (layers "F.Cu" "F.Mask") (roundrect_rratio 0.1) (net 16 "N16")
   (thermal_bridge_angle 45))
  (pad "13" thru_hole circle (at 7.62 -5.08) (size 1.524 1.524) (drill 0.889) (layers "*.Cu" "*.Mask") (remove_unused_layers no)
   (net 1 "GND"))
  (pad "13" smd roundrect (at 8.455 -5.08) (size 2.432 1.524) (layers "F.Cu" "F.Mask") (roundrect_rratio 0.1) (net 1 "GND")
   (thermal_bridge_angle 45))
  (pad "14" thru_hole circle (at 7.62 -7.62) (size 1.524 1.524) (drill 0.889) (layers "*.Cu" "*.Mask") (remove_unused_layers no)
   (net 5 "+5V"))
  (pad "14" smd roundrect (at 8.455 -7.62) (size 2.432 1.524) (layers "F.Cu" "F.Mask") (roundrect_rratio 0.1) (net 5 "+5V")
   (thermal_bridge_angle 45)))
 (gr_rect (start 175.26 90.424) (end 236.728 133.35) (stroke (width 0.05) (type solid)) (fill no) (layer "Edge.Cuts"))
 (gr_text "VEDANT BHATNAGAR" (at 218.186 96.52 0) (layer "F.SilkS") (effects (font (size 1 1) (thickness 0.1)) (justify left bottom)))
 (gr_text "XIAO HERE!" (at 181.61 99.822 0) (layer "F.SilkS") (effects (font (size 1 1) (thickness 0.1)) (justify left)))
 (segment (start 181.933 99.13681) (end 181.933 123.68747) (width 0.2) (layer "F.Cu") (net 4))
 (segment (start 227.34453 125.541) (end 232.89 119.99553) (width 0.2) (layer "F.Cu") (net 4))
 (segment (start 219.992 106.958) (end 207.5755 94.5415) (width 0.2) (layer "F.Cu") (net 4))
 (segment (start 186.52831 94.5415) (end 181.933 99.13681) (width 0.2) (layer "F.Cu") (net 4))
 (segment (start 181.933 123.68747) (end 183.78653 125.541) (width 0.2) (layer "F.Cu") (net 4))
 (segment (start 219.992 107.583) (end 219.992 106.958) (width 0.2) (layer "F.Cu") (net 4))
 (segment (start 183.78653 125.541) (end 227.34453 125.541) (width 0.2) (layer "F.Cu") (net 4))
 (segment (start 207.5755 94.5415) (end 186.52831 94.5415) (width 0.2) (layer "F.Cu") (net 4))
 (segment (start 232.89 119.99553) (end 232.89 109.333) (width 0.2) (layer "F.Cu") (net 4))
 (segment (start 175.702 105.1555) (end 177.219 103.6385) (width 0.2) (layer "F.Cu") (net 6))
 (segment (start 224.218 108.607) (end 233.991 108.607) (width 0.2) (layer "F.Cu") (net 6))
 (segment (start 183.62043 125.942) (end 175.702 118.02357) (width 0.2) (layer "F.Cu") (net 6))
 (segment (start 233.991 122.371) (end 230.42 125.942) (width 0.2) (layer "F.Cu") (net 6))
 (segment (start 230.42 125.942) (end 183.62043 125.942) (width 0.2) (layer "F.Cu") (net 6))
 (segment (start 175.702 118.02357) (end 175.702 105.1555) (width 0.2) (layer "F.Cu") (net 6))
 (segment (start 233.991 108.607) (end 233.991 122.371) (width 0.2) (layer "F.Cu") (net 6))
 (segment (start 223.492 109.333) (end 224.218 108.607) (width 0.2) (layer "F.Cu") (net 6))
 (segment (start 232.164 106.857) (end 232.89 107.583) (width 0.2) (layer "F.Cu") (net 5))
 (segment (start 223.492 107.583) (end 209.3875 93.4785) (width 0.2) (layer "F.Cu") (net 5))
 (segment (start 224.218 106.857) (end 232.164 106.857) (width 0.2) (layer "F.Cu") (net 5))
 (segment (start 209.3875 93.4785) (end 193.294 93.4785) (width 0.2) (layer "F.Cu") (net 5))
 (segment (start 223.492 107.583) (end 224.218 106.857) (width 0.2) (layer "F.Cu") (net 5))
 (segment (start 223.905 121.230314) (end 223.905 113.246) (width 0.2) (layer "F.Cu") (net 1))
 (segment (start 220.718 110.059) (end 219.992 109.333) (width 0.2) (layer "F.Cu") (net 1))
 (segment (start 205.2385 96.0185) (end 194.129 96.0185) (width 0.2) (layer "F.Cu") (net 1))
 (segment (start 219.992 109.333) (end 219.992 109.248) (width 0.2) (layer "F.Cu") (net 1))
 (segment (start 209.804 118.11) (end 207.975314 118.11) (width 0.2) (layer "F.Cu") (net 1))
 (segment (start 209.804 99.06) (end 208.28 99.06) (width 0.2) (layer "F.Cu") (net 1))
 (segment (start 228.854 109.869) (end 229.39 109.333) (width 0.2) (layer "F.Cu") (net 1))
 (segment (start 228.854 118.11) (end 228.854 109.869) (width 0.2) (layer "F.Cu") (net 1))
 (segment (start 223.084314 122.051) (end 223.905 121.230314) (width 0.2) (layer "F.Cu") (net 1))
 (segment (start 207.975314 118.11) (end 204.034314 122.051) (width 0.2) (layer "F.Cu") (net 1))
 (segment (start 223.905 113.246) (end 219.992 109.333) (width 0.2) (layer "F.Cu") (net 1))
 (segment (start 209.804 118.11) (end 212.924314 121.230314) (width 0.2) (layer "F.Cu") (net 1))
 (segment (start 221.923686 122.051) (end 223.084314 122.051) (width 0.2) (layer "F.Cu") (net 1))
 (segment (start 202.74347 122.051) (end 198.80247 118.11) (width 0.2) (layer "F.Cu") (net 1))
 (segment (start 204.034314 122.051) (end 202.74347 122.051) (width 0.2) (layer "F.Cu") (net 1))
 (segment (start 212.924314 121.230314) (end 221.103 121.230314) (width 0.2) (layer "F.Cu") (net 1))
 (segment (start 221.103 121.230314) (end 221.923686 122.051) (width 0.2) (layer "F.Cu") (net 1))
 (segment (start 228.664 110.059) (end 220.718 110.059) (width 0.2) (layer "F.Cu") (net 1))
 (segment (start 198.80247 118.11) (end 190.754 118.11) (width 0.2) (layer "F.Cu") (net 1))
 (segment (start 219.992 109.248) (end 209.804 99.06) (width 0.2) (layer "F.Cu") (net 1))
 (segment (start 208.28 99.06) (end 205.2385 96.0185) (width 0.2) (layer "F.Cu") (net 1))
 (segment (start 229.39 109.333) (end 228.664 110.059) (width 0.2) (layer "F.Cu") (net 1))
 (segment (start 183.003 109.88619) (end 183.003 121.230314) (width 0.2) (layer "F.Cu") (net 8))
 (segment (start 201.8895 100.0355) (end 192.85369 100.0355) (width 0.2) (layer "F.Cu") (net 8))
 (segment (start 184.984314 122.051) (end 185.805 121.230314) (width 0.2) (layer "F.Cu") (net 8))
 (segment (start 185.805 117.0425) (end 194.129 108.7185) (width 0.2) (layer "F.Cu") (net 8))
 (segment (start 203.454 101.6) (end 201.8895 100.0355) (width 0.2) (layer "F.Cu") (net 8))
 (segment (start 183.003 121.230314) (end 183.823686 122.051) (width 0.2) (layer "F.Cu") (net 8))
 (segment (start 183.823686 122.051) (end 184.984314 122.051) (width 0.2) (layer "F.Cu") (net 8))
 (segment (start 192.85369 100.0355) (end 183.003 109.88619) (width 0.2) (layer "F.Cu") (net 8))
 (segment (start 185.805 121.230314) (end 185.805 117.0425) (width 0.2) (layer "F.Cu") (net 8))
 (segment (start 203.454 120.65) (end 203.454 115.5035) (width 0.2) (layer "F.Cu") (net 7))
 (segment (start 203.454 115.5035) (end 194.129 106.1785) (width 0.2) (layer "F.Cu") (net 7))
 (segment (start 184.404 120.65) (end 184.404 113.3635) (width 0.2) (layer "F.Cu") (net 2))
 (segment (start 184.404 113.3635) (end 194.129 103.6385) (width 0.2) (layer "F.Cu") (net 2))
 (segment (start 222.504 120.65) (end 220.449184 120.65) (width 0.2) (layer "F.Cu") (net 9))
 (segment (start 220.449184 120.65) (end 200.897684 101.0985) (width 0.2) (layer "F.Cu") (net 9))
 (segment (start 200.897684 101.0985) (end 194.129 101.0985) (width 0.2) (layer "F.Cu") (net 9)))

